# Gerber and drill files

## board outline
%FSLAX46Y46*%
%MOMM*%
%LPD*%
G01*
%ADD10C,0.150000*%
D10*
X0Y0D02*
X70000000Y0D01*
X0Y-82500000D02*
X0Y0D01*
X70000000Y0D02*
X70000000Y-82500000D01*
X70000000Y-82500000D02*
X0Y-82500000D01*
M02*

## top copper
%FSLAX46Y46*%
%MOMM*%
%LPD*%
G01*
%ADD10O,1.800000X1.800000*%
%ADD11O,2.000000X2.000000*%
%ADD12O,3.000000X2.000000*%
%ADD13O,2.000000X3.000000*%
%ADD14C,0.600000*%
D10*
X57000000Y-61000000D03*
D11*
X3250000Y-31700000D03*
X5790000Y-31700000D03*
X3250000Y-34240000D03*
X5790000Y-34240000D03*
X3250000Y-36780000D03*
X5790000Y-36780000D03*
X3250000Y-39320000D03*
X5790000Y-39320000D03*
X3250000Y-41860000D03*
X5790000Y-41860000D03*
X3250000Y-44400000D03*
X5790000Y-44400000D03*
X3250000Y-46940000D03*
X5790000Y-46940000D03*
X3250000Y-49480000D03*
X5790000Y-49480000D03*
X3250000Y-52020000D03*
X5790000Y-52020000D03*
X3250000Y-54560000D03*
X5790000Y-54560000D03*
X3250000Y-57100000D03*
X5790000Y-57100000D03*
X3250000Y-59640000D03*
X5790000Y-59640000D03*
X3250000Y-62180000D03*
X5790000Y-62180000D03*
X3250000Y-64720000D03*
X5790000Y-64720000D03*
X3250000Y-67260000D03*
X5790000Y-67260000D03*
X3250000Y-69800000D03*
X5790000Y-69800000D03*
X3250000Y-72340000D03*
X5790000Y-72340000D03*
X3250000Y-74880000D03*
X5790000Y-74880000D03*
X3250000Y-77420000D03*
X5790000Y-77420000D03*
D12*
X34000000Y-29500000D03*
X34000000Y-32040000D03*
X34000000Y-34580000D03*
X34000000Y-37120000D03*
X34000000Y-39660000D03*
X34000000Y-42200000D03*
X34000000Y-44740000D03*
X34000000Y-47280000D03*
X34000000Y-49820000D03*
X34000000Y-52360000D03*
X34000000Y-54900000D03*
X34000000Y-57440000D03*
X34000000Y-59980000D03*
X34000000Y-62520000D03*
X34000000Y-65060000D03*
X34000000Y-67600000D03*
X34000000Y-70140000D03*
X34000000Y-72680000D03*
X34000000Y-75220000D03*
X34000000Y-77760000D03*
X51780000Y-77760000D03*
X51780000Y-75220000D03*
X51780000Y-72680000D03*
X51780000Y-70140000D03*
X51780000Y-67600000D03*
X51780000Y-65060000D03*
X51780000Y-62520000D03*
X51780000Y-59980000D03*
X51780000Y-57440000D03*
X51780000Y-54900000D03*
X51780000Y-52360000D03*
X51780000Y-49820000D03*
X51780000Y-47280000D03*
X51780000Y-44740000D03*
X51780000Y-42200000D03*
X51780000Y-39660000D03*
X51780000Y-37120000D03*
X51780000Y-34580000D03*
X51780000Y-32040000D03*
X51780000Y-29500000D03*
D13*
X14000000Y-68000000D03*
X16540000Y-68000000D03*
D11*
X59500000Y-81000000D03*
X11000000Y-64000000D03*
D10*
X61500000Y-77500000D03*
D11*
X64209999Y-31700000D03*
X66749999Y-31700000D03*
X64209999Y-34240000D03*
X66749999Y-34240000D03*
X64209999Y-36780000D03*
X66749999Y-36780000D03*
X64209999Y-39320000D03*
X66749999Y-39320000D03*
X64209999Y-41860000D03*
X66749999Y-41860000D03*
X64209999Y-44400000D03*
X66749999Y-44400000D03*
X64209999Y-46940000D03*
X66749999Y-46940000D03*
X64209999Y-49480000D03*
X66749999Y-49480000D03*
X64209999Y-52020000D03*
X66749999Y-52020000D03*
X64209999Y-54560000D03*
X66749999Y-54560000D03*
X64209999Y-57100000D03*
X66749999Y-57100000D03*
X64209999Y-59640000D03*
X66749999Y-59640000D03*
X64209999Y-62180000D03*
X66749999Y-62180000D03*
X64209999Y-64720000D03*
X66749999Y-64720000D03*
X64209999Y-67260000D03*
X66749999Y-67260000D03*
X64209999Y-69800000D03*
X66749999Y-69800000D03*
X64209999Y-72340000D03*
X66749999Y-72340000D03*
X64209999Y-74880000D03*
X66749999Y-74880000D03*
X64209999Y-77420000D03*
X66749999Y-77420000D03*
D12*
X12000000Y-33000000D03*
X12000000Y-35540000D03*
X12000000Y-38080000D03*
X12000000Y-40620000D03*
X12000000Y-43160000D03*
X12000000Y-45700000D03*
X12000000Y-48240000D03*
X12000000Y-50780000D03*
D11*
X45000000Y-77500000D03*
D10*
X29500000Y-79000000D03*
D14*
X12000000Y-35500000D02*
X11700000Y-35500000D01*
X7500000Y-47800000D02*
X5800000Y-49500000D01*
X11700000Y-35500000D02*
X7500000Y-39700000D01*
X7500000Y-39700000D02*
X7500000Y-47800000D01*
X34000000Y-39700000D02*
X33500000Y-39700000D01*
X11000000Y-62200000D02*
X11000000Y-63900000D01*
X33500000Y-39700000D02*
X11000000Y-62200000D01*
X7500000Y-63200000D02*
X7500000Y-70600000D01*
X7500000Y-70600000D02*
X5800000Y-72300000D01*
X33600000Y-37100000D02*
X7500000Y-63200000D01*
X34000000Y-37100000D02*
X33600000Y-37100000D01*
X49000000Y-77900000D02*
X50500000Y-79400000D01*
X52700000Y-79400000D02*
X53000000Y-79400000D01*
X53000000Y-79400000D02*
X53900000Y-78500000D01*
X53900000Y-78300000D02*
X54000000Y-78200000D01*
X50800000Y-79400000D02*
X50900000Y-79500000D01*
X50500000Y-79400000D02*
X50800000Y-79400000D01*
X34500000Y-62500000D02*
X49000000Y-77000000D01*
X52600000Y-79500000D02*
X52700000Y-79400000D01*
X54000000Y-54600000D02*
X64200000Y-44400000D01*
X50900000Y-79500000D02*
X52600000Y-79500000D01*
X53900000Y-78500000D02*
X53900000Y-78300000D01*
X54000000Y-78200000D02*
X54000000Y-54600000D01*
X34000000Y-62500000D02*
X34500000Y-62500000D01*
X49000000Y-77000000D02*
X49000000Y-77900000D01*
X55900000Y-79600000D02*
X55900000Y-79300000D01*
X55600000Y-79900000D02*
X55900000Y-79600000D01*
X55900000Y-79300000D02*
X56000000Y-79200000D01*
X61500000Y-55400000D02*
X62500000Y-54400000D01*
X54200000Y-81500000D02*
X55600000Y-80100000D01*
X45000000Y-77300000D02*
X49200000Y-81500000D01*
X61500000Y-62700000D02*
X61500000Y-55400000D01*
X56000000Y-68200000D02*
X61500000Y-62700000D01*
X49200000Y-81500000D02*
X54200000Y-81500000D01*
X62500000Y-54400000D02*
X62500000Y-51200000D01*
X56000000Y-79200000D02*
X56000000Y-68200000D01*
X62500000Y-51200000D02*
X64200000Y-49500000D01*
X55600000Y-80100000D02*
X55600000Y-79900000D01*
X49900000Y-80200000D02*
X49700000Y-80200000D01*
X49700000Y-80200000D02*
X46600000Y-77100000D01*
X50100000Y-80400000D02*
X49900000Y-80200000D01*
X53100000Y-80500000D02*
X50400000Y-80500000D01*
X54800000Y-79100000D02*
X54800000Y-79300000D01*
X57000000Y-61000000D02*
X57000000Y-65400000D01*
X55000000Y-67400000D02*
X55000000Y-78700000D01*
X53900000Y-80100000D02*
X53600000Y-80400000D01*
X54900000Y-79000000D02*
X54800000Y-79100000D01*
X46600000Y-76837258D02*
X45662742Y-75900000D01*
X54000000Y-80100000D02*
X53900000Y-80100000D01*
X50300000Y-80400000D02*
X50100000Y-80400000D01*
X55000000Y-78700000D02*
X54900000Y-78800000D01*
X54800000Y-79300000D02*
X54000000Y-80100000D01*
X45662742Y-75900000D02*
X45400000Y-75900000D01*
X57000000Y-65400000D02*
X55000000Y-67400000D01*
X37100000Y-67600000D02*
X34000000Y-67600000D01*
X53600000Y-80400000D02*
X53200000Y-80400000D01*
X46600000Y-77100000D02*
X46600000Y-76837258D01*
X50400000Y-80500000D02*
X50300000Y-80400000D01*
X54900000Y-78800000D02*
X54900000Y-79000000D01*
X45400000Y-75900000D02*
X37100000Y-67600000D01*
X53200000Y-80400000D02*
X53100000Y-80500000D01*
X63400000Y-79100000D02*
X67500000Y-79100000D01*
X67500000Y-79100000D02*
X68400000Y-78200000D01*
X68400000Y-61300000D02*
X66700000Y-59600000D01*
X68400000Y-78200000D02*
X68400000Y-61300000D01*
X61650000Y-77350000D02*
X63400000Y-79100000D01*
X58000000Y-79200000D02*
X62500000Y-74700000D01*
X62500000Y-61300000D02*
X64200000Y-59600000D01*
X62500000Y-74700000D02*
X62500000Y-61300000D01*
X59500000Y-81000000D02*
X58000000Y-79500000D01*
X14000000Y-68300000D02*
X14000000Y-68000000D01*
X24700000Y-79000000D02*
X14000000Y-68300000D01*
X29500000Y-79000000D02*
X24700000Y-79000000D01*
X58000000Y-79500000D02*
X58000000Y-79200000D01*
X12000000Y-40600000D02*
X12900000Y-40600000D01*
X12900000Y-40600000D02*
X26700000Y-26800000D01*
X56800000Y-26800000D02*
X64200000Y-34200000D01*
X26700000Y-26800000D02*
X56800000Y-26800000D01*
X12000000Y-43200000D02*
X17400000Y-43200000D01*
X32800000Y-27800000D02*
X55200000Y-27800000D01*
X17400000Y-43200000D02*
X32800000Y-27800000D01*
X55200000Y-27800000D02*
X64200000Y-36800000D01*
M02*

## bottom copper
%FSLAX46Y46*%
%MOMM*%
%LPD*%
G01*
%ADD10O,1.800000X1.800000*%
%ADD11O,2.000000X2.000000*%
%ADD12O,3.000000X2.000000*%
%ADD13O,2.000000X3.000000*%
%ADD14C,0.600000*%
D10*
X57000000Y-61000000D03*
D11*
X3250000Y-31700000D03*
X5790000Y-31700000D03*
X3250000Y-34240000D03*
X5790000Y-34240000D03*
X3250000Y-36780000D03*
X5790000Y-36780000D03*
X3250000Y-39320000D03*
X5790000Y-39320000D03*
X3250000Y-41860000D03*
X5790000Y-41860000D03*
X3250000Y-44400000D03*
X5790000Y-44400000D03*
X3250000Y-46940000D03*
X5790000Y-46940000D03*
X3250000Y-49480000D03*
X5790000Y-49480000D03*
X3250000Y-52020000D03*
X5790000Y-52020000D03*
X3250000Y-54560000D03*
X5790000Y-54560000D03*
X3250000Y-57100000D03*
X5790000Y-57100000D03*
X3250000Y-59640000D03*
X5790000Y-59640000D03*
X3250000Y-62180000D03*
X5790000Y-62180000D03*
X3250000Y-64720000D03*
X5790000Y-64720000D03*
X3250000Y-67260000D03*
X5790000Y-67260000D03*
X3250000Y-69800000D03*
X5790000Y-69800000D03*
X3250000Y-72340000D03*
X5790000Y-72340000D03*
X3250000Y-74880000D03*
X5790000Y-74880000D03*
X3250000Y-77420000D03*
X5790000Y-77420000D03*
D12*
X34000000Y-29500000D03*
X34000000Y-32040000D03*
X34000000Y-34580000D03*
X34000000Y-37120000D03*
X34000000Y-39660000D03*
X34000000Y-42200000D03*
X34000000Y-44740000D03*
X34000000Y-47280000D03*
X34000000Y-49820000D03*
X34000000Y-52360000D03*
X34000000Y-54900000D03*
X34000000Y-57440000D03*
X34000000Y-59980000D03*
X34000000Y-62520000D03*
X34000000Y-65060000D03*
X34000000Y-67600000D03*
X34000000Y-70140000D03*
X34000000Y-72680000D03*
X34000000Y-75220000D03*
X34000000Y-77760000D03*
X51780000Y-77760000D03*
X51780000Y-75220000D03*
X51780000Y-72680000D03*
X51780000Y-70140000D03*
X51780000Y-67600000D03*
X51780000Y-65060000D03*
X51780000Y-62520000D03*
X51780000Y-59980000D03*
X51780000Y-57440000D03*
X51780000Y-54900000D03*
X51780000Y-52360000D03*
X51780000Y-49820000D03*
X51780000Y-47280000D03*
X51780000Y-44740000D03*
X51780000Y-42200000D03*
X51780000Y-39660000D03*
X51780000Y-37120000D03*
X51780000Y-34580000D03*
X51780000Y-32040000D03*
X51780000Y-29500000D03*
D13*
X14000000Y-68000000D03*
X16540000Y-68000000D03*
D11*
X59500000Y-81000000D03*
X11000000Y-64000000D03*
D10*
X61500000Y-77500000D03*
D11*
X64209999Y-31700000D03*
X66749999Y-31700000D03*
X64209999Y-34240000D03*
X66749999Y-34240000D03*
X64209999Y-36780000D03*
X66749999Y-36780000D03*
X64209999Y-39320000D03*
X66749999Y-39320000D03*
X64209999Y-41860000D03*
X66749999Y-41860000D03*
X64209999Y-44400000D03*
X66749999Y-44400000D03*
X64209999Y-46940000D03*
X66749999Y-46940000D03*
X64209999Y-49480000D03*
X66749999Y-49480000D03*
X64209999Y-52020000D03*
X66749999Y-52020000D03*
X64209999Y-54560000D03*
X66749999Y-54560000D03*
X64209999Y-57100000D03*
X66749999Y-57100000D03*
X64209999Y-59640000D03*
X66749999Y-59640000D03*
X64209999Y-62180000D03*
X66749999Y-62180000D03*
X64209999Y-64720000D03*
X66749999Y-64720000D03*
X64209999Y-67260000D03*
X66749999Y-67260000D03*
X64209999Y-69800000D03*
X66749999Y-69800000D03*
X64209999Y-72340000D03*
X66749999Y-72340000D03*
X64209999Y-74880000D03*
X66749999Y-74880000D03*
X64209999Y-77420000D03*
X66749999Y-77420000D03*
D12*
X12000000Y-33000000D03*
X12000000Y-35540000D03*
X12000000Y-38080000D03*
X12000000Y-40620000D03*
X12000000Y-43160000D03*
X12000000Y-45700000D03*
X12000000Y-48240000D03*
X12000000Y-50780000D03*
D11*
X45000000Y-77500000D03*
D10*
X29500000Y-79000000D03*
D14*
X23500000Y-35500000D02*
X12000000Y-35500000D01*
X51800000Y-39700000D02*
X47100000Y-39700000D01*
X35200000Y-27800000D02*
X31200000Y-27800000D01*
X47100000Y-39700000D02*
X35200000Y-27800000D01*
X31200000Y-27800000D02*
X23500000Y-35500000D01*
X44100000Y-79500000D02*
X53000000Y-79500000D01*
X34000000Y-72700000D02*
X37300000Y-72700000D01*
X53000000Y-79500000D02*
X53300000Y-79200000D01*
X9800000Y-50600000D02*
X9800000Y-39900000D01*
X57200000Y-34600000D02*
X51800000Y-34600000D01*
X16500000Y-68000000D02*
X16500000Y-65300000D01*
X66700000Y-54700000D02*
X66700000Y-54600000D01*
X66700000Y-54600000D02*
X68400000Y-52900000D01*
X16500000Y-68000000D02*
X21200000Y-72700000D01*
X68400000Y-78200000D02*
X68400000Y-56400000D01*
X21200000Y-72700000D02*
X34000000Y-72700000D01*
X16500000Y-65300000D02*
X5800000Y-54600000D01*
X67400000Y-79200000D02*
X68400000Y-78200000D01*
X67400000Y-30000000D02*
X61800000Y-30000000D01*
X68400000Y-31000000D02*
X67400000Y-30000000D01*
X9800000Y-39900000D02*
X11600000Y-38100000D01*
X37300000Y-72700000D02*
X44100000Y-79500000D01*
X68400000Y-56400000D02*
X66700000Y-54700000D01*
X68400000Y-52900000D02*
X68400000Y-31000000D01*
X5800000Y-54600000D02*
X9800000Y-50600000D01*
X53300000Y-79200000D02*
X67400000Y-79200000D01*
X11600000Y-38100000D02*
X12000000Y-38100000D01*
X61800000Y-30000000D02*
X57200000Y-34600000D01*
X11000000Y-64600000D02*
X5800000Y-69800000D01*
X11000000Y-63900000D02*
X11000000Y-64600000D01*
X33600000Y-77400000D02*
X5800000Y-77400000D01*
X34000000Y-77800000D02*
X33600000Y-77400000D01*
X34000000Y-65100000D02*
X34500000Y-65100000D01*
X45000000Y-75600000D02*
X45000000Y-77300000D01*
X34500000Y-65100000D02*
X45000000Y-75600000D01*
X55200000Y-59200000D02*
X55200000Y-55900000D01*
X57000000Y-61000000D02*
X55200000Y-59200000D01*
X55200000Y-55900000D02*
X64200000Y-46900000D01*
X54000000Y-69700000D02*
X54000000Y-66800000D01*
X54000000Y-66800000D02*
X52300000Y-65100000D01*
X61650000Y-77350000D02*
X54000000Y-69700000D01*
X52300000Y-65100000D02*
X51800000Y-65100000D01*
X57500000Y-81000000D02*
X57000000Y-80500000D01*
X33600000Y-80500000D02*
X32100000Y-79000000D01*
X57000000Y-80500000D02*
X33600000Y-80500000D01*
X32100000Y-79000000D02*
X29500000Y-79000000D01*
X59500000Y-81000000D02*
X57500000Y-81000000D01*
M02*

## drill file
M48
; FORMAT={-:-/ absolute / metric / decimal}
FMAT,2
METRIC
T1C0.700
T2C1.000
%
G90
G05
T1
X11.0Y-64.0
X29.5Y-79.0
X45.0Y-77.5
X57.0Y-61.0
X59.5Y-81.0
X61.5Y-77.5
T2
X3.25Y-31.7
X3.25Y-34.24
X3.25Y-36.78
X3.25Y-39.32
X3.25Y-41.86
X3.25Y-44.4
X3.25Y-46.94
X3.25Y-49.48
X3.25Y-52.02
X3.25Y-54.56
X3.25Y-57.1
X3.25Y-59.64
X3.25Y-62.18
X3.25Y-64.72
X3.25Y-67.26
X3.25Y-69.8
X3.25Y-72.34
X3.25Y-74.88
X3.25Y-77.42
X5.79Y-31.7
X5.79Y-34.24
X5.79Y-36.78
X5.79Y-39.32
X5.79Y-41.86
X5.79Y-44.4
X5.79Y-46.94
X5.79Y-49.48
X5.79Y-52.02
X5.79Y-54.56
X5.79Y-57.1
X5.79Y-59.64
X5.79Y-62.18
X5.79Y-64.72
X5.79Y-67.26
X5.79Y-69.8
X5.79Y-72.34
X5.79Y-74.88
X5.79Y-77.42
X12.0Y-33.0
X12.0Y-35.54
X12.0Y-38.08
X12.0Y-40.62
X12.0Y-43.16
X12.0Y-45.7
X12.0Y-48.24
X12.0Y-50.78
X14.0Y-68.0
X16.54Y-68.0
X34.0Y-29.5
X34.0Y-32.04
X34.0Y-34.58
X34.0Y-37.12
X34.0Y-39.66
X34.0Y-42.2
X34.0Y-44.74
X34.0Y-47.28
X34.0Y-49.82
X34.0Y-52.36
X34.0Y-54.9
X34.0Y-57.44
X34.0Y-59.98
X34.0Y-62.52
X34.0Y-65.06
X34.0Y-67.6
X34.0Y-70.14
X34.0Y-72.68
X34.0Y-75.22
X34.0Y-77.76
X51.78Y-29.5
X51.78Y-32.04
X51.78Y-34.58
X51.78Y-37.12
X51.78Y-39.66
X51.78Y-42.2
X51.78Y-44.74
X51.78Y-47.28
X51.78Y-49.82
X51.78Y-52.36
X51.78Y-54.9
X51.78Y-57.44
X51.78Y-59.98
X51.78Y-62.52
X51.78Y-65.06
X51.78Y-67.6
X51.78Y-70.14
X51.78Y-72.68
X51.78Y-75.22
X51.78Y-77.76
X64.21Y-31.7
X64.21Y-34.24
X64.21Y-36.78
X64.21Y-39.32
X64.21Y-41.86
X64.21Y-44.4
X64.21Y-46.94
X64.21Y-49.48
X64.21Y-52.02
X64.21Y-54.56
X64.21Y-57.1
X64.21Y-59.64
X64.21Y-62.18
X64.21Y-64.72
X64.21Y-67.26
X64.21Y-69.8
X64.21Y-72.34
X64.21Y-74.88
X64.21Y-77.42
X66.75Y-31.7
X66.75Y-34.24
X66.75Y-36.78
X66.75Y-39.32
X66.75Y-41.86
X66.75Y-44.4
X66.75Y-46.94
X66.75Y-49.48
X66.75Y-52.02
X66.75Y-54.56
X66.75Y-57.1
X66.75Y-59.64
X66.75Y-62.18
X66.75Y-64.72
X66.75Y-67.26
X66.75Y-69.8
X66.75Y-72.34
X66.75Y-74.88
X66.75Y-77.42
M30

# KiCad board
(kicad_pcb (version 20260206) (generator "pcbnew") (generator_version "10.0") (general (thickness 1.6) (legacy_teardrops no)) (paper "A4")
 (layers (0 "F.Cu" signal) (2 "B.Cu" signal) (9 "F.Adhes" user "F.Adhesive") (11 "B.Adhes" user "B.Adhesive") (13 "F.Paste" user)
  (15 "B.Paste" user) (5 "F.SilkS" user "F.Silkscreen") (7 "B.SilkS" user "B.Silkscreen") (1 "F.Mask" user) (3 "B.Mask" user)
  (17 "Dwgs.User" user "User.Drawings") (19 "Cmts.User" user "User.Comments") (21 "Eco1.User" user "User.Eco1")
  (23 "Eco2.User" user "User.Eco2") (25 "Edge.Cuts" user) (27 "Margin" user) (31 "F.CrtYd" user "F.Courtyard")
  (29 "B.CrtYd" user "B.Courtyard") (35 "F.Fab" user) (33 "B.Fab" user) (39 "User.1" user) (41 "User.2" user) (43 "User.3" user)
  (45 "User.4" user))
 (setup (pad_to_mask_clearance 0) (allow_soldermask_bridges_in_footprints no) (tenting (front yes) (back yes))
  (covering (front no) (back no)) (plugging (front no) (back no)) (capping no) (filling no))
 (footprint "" (layer "F.Cu") (at 57 61)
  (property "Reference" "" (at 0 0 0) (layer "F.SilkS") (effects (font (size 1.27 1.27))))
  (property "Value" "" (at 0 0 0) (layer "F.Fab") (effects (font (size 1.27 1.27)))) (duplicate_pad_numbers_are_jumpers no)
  (pad "2" thru_hole oval (at 0 0) (size 1.8 1.8) (drill 0.7) (layers "*.Cu" "*.Mask") (remove_unused_layers no)))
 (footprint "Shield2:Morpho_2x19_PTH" (layer "F.Cu") (at 3.25 31.7)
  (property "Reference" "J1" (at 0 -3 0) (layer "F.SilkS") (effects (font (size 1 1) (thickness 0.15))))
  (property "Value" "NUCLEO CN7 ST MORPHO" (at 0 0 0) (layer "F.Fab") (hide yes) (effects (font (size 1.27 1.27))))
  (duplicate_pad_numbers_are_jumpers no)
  (pad "1" thru_hole oval (at 0 0) (size 2 2) (drill 1) (layers "*.Cu") (remove_unused_layers no) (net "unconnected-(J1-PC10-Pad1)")
   (thermal_bridge_angle 45))
  (pad "2" thru_hole oval (at 2.54 0) (size 2 2) (drill 1) (layers "*.Cu") (remove_unused_layers no) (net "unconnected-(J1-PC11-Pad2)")
   (thermal_bridge_angle 45))
  (pad "3" thru_hole oval (at 0 2.54) (size 2 2) (drill 1) (layers "*.Cu") (remove_unused_layers no) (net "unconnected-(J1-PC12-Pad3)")
   (thermal_bridge_angle 45))
  (pad "4" thru_hole oval (at 2.54 2.54) (size 2 2) (drill 1) (layers "*.Cu") (remove_unused_layers no) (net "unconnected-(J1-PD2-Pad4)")
   (thermal_bridge_angle 45))
  (pad "5" thru_hole oval (at 0 5.08) (size 2 2) (drill 1) (layers "*.Cu") (remove_unused_layers no) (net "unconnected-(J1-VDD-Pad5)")
   (thermal_bridge_angle 45))
  (pad "6" thru_hole oval (at 2.54 5.08) (size 2 2) (drill 1) (layers "*.Cu") (remove_unused_layers no) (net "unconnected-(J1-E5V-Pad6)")
   (thermal_bridge_angle 45))
  (pad "7" thru_hole oval (at 0 7.62) (size 2 2) (drill 1) (layers "*.Cu") (remove_unused_layers no) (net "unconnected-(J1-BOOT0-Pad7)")
   (thermal_bridge_angle 45))
  (pad "8" thru_hole oval (at 2.54 7.62) (size 2 2) (drill 1) (layers "*.Cu") (remove_unused_layers no) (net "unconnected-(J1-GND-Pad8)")
   (thermal_bridge_angle 45))
  (pad "9" thru_hole oval (at 0 10.16) (size 2 2) (drill 1) (layers "*.Cu") (remove_unused_layers no) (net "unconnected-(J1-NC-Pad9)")
   (thermal_bridge_angle 45))
  (pad "10" thru_hole oval (at 2.54 10.16) (size 2 2) (drill 1) (layers "*.Cu") (remove_unused_layers no) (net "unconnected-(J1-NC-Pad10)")
   (thermal_bridge_angle 45))
  (pad "11" thru_hole oval (at 0 12.7) (size 2 2) (drill 1) (layers "*.Cu") (remove_unused_layers no) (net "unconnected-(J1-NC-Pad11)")
   (thermal_bridge_angle 45))
  (pad "12" thru_hole oval (at 2.54 12.7) (size 2 2) (drill 1) (layers "*.Cu") (remove_unused_layers no)
   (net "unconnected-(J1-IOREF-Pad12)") (thermal_bridge_angle 45))
  (pad "13" thru_hole oval (at 0 15.24) (size 2 2) (drill 1) (layers "*.Cu") (remove_unused_layers no) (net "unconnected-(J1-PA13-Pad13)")
   (thermal_bridge_angle 45))
  (pad "14" thru_hole oval (at 2.54 15.24) (size 2 2) (drill 1) (layers "*.Cu") (remove_unused_layers no)
   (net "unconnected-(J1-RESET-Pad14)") (thermal_bridge_angle 45))
  (pad "15" thru_hole oval (at 0 17.78) (size 2 2) (drill 1) (layers "*.Cu") (remove_unused_layers no) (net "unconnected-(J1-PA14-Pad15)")
   (thermal_bridge_angle 45))
  (pad "16" thru_hole oval (at 2.54 17.78) (size 2 2) (drill 1) (layers "*.Cu") (remove_unused_layers no) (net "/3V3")
   (thermal_bridge_angle 45))
  (pad "17" thru_hole oval (at 0 20.32) (size 2 2) (drill 1) (layers "*.Cu") (remove_unused_layers no) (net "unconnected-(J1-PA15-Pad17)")
   (thermal_bridge_angle 45))
  (pad "18" thru_hole oval (at 2.54 20.32) (size 2 2) (drill 1) (layers "*.Cu") (remove_unused_layers no) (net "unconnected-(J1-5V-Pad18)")
   (thermal_bridge_angle 45))
  (pad "19" thru_hole oval (at 0 22.86) (size 2 2) (drill 1) (layers "*.Cu") (remove_unused_layers no) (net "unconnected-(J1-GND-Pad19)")
   (thermal_bridge_angle 45))
  (pad "20" thru_hole oval (at 2.54 22.86) (size 2 2) (drill 1) (layers "*.Cu") (remove_unused_layers no) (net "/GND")
   (thermal_bridge_angle 45))
  (pad "21" thru_hole oval (at 0 25.4) (size 2 2) (drill 1) (layers "*.Cu") (remove_unused_layers no) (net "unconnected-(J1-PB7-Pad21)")
   (thermal_bridge_angle 45))
  (pad "22" thru_hole oval (at 2.54 25.4) (size 2 2) (drill 1) (layers "*.Cu") (remove_unused_layers no) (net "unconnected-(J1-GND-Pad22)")
   (thermal_bridge_angle 45))
  (pad "23" thru_hole oval (at 0 27.94) (size 2 2) (drill 1) (layers "*.Cu") (remove_unused_layers no) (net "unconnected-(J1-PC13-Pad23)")
   (thermal_bridge_angle 45))
  (pad "24" thru_hole oval (at 2.54 27.94) (size 2 2) (drill 1) (layers "*.Cu") (remove_unused_layers no) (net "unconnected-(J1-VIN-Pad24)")
   (thermal_bridge_angle 45))
  (pad "25" thru_hole oval (at 0 30.48) (size 2 2) (drill 1) (layers "*.Cu") (remove_unused_layers no) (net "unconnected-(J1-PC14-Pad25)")
   (thermal_bridge_angle 45))
  (pad "26" thru_hole oval (at 2.54 30.48) (size 2 2) (drill 1) (layers "*.Cu") (remove_unused_layers no) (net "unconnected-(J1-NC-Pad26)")
   (thermal_bridge_angle 45))
  (pad "27" thru_hole oval (at 0 33.02) (size 2 2) (drill 1) (layers "*.Cu") (remove_unused_layers no) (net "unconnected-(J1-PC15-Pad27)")
   (thermal_bridge_angle 45))
  (pad "28" thru_hole oval (at 2.54 33.02) (size 2 2) (drill 1) (layers "*.Cu") (remove_unused_layers no) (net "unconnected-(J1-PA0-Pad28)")
   (thermal_bridge_angle 45))
  (pad "29" thru_hole oval (at 0 35.56) (size 2 2) (drill 1) (layers "*.Cu") (remove_unused_layers no) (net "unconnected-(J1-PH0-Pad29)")
   (thermal_bridge_angle 45))
  (pad "30" thru_hole oval (at 2.54 35.56) (size 2 2) (drill 1) (layers "*.Cu") (remove_unused_layers no) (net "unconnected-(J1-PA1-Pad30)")
   (thermal_bridge_angle 45))
  (pad "31" thru_hole oval (at 0 38.1) (size 2 2) (drill 1) (layers "*.Cu") (remove_unused_layers no) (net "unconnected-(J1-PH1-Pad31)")
   (thermal_bridge_angle 45))
  (pad "32" thru_hole oval (at 2.54 38.1) (size 2 2) (drill 1) (layers "*.Cu") (remove_unused_layers no) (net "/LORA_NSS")
   (thermal_bridge_angle 45))
  (pad "33" thru_hole oval (at 0 40.64) (size 2 2) (drill 1) (layers "*.Cu") (remove_unused_layers no) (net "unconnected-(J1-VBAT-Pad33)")
   (thermal_bridge_angle 45))
  (pad "34" thru_hole oval (at 2.54 40.64) (size 2 2) (drill 1) (layers "*.Cu") (remove_unused_layers no) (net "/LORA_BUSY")
   (thermal_bridge_angle 45))
  (pad "35" thru_hole oval (at 0 43.18) (size 2 2) (drill 1) (layers "*.Cu") (remove_unused_layers no) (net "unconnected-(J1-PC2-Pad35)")
   (thermal_bridge_angle 45))
  (pad "36" thru_hole oval (at 2.54 43.18) (size 2 2) (drill 1) (layers "*.Cu") (remove_unused_layers no)
   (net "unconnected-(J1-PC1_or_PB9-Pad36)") (thermal_bridge_angle 45))
  (pad "37" thru_hole oval (at 0 45.72) (size 2 2) (drill 1) (layers "*.Cu") (remove_unused_layers no) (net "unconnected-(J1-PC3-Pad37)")
   (thermal_bridge_angle 45))
  (pad "38" thru_hole oval (at 2.54 45.72) (size 2 2) (drill 1) (layers "*.Cu") (remove_unused_layers no) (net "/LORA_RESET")
   (thermal_bridge_angle 45)))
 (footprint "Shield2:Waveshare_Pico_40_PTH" (layer "F.Cu") (at 34 29.5)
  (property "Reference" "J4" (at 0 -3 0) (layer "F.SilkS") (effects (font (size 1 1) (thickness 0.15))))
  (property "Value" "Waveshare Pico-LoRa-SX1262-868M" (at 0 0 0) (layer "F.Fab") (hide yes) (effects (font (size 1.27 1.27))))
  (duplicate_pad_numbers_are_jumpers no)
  (pad "1" thru_hole oval (at 0 0) (size 3 2) (drill 1) (layers "*.Cu") (remove_unused_layers no) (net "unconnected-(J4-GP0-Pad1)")
   (thermal_bridge_angle 45))
  (pad "2" thru_hole oval (at 0 2.54) (size 3 2) (drill 1) (layers "*.Cu") (remove_unused_layers no) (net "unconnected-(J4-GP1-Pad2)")
   (thermal_bridge_angle 45))
  (pad "3" thru_hole oval (at 0 5.08) (size 3 2) (drill 1) (layers "*.Cu") (remove_unused_layers no) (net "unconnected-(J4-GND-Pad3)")
   (thermal_bridge_angle 45))
  (pad "4" thru_hole oval (at 0 7.62) (size 3 2) (drill 1) (layers "*.Cu") (remove_unused_layers no) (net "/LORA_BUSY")
   (thermal_bridge_angle 45))
  (pad "5" thru_hole oval (at 0 10.16) (size 3 2) (drill 1) (layers "*.Cu") (remove_unused_layers no) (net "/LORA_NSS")
   (thermal_bridge_angle 45))
  (pad "6" thru_hole oval (at 0 12.7) (size 3 2) (drill 1) (layers "*.Cu") (remove_unused_layers no) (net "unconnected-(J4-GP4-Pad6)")
   (thermal_bridge_angle 45))
  (pad "7" thru_hole oval (at 0 15.24) (size 3 2) (drill 1) (layers "*.Cu") (remove_unused_layers no) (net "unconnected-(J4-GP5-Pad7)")
   (thermal_bridge_angle 45))
  (pad "8" thru_hole oval (at 0 17.78) (size 3 2) (drill 1) (layers "*.Cu") (remove_unused_layers no) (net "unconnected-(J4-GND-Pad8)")
   (thermal_bridge_angle 45))
  (pad "9" thru_hole oval (at 0 20.32) (size 3 2) (drill 1) (layers "*.Cu") (remove_unused_layers no) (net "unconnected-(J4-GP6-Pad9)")
   (thermal_bridge_angle 45))
  (pad "10" thru_hole oval (at 0 22.86) (size 3 2) (drill 1) (layers "*.Cu") (remove_unused_layers no) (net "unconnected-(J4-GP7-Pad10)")
   (thermal_bridge_angle 45))
  (pad "11" thru_hole oval (at 0 25.4) (size 3 2) (drill 1) (layers "*.Cu") (remove_unused_layers no) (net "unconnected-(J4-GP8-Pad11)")
   (thermal_bridge_angle 45))
  (pad "12" thru_hole oval (at 0 27.94) (size 3 2) (drill 1) (layers "*.Cu") (remove_unused_layers no) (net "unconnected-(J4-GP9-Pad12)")
   (thermal_bridge_angle 45))
  (pad "13" thru_hole oval (at 0 30.48) (size 3 2) (drill 1) (layers "*.Cu") (remove_unused_layers no) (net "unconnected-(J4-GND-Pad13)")
   (thermal_bridge_angle 45))
  (pad "14" thru_hole oval (at 0 33.02) (size 3 2) (drill 1) (layers "*.Cu") (remove_unused_layers no) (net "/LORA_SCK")
   (thermal_bridge_angle 45))
  (pad "15" thru_hole oval (at 0 35.56) (size 3 2) (drill 1) (layers "*.Cu") (remove_unused_layers no) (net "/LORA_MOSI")
   (thermal_bridge_angle 45))
  (pad "16" thru_hole oval (at 0 38.1) (size 3 2) (drill 1) (layers "*.Cu") (remove_unused_layers no) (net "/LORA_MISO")
   (thermal_bridge_angle 45))
  (pad "17" thru_hole oval (at 0 40.64) (size 3 2) (drill 1) (layers "*.Cu") (remove_unused_layers no) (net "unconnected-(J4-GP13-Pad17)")
   (thermal_bridge_angle 45))
  (pad "18" thru_hole oval (at 0 43.18) (size 3 2) (drill 1) (layers "*.Cu") (remove_unused_layers no) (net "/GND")
   (thermal_bridge_angle 45))
  (pad "19" thru_hole oval (at 0 45.72) (size 3 2) (drill 1) (layers "*.Cu") (remove_unused_layers no) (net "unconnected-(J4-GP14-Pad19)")
   (thermal_bridge_angle 45))
  (pad "20" thru_hole oval (at 0 48.26) (size 3 2) (drill 1) (layers "*.Cu") (remove_unused_layers no) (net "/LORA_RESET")
   (thermal_bridge_angle 45))
  (pad "21" thru_hole oval (at 17.78 48.26) (size 3 2) (drill 1) (layers "*.Cu") (remove_unused_layers no)
   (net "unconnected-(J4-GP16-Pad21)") (thermal_bridge_angle 45))
  (pad "22" thru_hole oval (at 17.78 45.72) (size 3 2) (drill 1) (layers "*.Cu") (remove_unused_layers no)
   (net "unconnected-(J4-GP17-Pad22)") (thermal_bridge_angle 45))
  (pad "23" thru_hole oval (at 17.78 43.18) (size 3 2) (drill 1) (layers "*.Cu") (remove_unused_layers no)
   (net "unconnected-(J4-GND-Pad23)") (thermal_bridge_angle 45))
  (pad "24" thru_hole oval (at 17.78 40.64) (size 3 2) (drill 1) (layers "*.Cu") (remove_unused_layers no)
   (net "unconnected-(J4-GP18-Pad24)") (thermal_bridge_angle 45))
  (pad "25" thru_hole oval (at 17.78 38.1) (size 3 2) (drill 1) (layers "*.Cu") (remove_unused_layers no)
   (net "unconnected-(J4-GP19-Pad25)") (thermal_bridge_angle 45))
  (pad "26" thru_hole oval (at 17.78 35.56) (size 3 2) (drill 1) (layers "*.Cu") (remove_unused_layers no) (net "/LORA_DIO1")
   (thermal_bridge_angle 45))
  (pad "27" thru_hole oval (at 17.78 33.02) (size 3 2) (drill 1) (layers "*.Cu") (remove_unused_layers no)
   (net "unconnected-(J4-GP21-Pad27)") (thermal_bridge_angle 45))
  (pad "28" thru_hole oval (at 17.78 30.48) (size 3 2) (drill 1) (layers "*.Cu") (remove_unused_layers no)
   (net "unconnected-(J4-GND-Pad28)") (thermal_bridge_angle 45))
  (pad "29" thru_hole oval (at 17.78 27.94) (size 3 2) (drill 1) (layers "*.Cu") (remove_unused_layers no)
   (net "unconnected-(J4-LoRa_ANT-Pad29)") (thermal_bridge_angle 45))
  (pad "30" thru_hole oval (at 17.78 25.4) (size 3 2) (drill 1) (layers "*.Cu") (remove_unused_layers no) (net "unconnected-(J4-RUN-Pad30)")
   (thermal_bridge_angle 45))
  (pad "31" thru_hole oval (at 17.78 22.86) (size 3 2) (drill 1) (layers "*.Cu") (remove_unused_layers no)
   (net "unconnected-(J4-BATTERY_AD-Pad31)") (thermal_bridge_angle 45))
  (pad "32" thru_hole oval (at 17.78 20.32) (size 3 2) (drill 1) (layers "*.Cu") (remove_unused_layers no)
   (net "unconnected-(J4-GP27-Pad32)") (thermal_bridge_angle 45))
  (pad "33" thru_hole oval (at 17.78 17.78) (size 3 2) (drill 1) (layers "*.Cu") (remove_unused_layers no)
   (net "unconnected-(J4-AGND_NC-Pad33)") (thermal_bridge_angle 45))
  (pad "34" thru_hole oval (at 17.78 15.24) (size 3 2) (drill 1) (layers "*.Cu") (remove_unused_layers no)
   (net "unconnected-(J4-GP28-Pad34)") (thermal_bridge_angle 45))
  (pad "35" thru_hole oval (at 17.78 12.7) (size 3 2) (drill 1) (layers "*.Cu") (remove_unused_layers no)
   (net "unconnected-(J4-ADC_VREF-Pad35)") (thermal_bridge_angle 45))
  (pad "36" thru_hole oval (at 17.78 10.16) (size 3 2) (drill 1) (layers "*.Cu") (remove_unused_layers no) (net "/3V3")
   (thermal_bridge_angle 45))
  (pad "37" thru_hole oval (at 17.78 7.62) (size 3 2) (drill 1) (layers "*.Cu") (remove_unused_layers no)
   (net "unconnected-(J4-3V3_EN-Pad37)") (thermal_bridge_angle 45))
  (pad "38" thru_hole oval (at 17.78 5.08) (size 3 2) (drill 1) (layers "*.Cu") (remove_unused_layers no) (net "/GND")
   (thermal_bridge_angle 45))
  (pad "39" thru_hole oval (at 17.78 2.54) (size 3 2) (drill 1) (layers "*.Cu") (remove_unused_layers no)
   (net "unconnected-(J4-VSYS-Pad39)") (thermal_bridge_angle 45))
  (pad "40" thru_hole oval (at 17.78 0) (size 3 2) (drill 1) (layers "*.Cu") (remove_unused_layers no) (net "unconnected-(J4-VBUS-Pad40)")
   (thermal_bridge_angle 45)))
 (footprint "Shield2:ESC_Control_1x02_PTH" (layer "F.Cu") (at 14 68)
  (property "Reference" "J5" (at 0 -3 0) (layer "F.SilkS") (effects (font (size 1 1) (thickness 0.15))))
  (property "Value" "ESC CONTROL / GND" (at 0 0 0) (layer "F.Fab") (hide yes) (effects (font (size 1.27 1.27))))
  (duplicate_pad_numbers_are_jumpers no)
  (pad "1" thru_hole oval (at 0 0) (size 2 3) (drill 1) (layers "*.Cu") (remove_unused_layers no) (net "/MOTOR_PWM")
   (thermal_bridge_angle 45))
  (pad "2" thru_hole oval (at 2.54 0) (size 2 3) (drill 1) (layers "*.Cu") (remove_unused_layers no) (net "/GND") (thermal_bridge_angle 45)))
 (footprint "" (layer "F.Cu") (at 59.5 81)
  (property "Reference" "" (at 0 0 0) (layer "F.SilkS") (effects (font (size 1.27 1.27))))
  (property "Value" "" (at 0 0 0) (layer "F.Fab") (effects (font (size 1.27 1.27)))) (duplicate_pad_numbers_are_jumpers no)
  (pad "2" thru_hole oval (at 0 0) (size 2 2) (drill 0.7) (layers "*.Cu" "*.Mask") (remove_unused_layers no)))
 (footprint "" (layer "F.Cu") (at 11 64)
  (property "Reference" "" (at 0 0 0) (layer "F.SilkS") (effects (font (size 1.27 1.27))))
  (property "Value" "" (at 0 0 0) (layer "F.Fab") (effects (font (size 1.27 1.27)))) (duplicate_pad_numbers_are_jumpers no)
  (pad "2" thru_hole oval (at 0 0) (size 2 2) (drill 0.7) (layers "*.Cu" "*.Mask") (remove_unused_layers no)))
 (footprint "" (layer "F.Cu") (at 61.5 77.5)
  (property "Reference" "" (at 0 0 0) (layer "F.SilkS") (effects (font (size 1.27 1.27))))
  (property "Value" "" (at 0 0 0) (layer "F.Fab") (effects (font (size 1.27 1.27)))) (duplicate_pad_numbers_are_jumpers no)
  (pad "2" thru_hole oval (at 0 0) (size 1.8 1.8) (drill 0.7) (layers "*.Cu" "*.Mask") (remove_unused_layers no)))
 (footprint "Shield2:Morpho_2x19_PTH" (layer "F.Cu") (at 64.209999 31.7)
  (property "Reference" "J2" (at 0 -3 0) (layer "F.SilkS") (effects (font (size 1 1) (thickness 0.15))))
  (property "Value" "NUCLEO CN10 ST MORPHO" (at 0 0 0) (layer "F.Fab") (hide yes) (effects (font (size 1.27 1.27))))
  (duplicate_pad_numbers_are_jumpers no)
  (pad "1" thru_hole oval (at 0 0) (size 2 2) (drill 1) (layers "*.Cu") (remove_unused_layers no) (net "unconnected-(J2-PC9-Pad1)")
   (thermal_bridge_angle 45))
  (pad "2" thru_hole oval (at 2.54 0) (size 2 2) (drill 1) (layers "*.Cu") (remove_unused_layers no) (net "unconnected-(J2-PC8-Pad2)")
   (thermal_bridge_angle 45))
  (pad "3" thru_hole oval (at 0 2.54) (size 2 2) (drill 1) (layers "*.Cu") (remove_unused_layers no) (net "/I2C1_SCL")
   (thermal_bridge_angle 45))
  (pad "4" thru_hole oval (at 2.54 2.54) (size 2 2) (drill 1) (layers "*.Cu") (remove_unused_layers no) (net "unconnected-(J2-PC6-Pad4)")
   (thermal_bridge_angle 45))
  (pad "5" thru_hole oval (at 0 5.08) (size 2 2) (drill 1) (layers "*.Cu") (remove_unused_layers no) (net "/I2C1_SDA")
   (thermal_bridge_angle 45))
  (pad "6" thru_hole oval (at 2.54 5.08) (size 2 2) (drill 1) (layers "*.Cu") (remove_unused_layers no) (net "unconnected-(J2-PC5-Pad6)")
   (thermal_bridge_angle 45))
  (pad "7" thru_hole oval (at 0 7.62) (size 2 2) (drill 1) (layers "*.Cu") (remove_unused_layers no) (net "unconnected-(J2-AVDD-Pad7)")
   (thermal_bridge_angle 45))
  (pad "8" thru_hole oval (at 2.54 7.62) (size 2 2) (drill 1) (layers "*.Cu") (remove_unused_layers no) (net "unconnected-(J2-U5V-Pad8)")
   (thermal_bridge_angle 45))
  (pad "9" thru_hole oval (at 0 10.16) (size 2 2) (drill 1) (layers "*.Cu") (remove_unused_layers no) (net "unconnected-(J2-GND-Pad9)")
   (thermal_bridge_angle 45))
  (pad "10" thru_hole oval (at 2.54 10.16) (size 2 2) (drill 1) (layers "*.Cu") (remove_unused_layers no) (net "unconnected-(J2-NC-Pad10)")
   (thermal_bridge_angle 45))
  (pad "11" thru_hole oval (at 0 12.7) (size 2 2) (drill 1) (layers "*.Cu") (remove_unused_layers no) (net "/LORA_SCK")
   (thermal_bridge_angle 45))
  (pad "12" thru_hole oval (at 2.54 12.7) (size 2 2) (drill 1) (layers "*.Cu") (remove_unused_layers no) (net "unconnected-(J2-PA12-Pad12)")
   (thermal_bridge_angle 45))
  (pad "13" thru_hole oval (at 0 15.24) (size 2 2) (drill 1) (layers "*.Cu") (remove_unused_layers no) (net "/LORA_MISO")
   (thermal_bridge_angle 45))
  (pad "14" thru_hole oval (at 2.54 15.24) (size 2 2) (drill 1) (layers "*.Cu") (remove_unused_layers no)
   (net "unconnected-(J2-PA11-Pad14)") (thermal_bridge_angle 45))
  (pad "15" thru_hole oval (at 0 17.78) (size 2 2) (drill 1) (layers "*.Cu") (remove_unused_layers no) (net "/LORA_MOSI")
   (thermal_bridge_angle 45))
  (pad "16" thru_hole oval (at 2.54 17.78) (size 2 2) (drill 1) (layers "*.Cu") (remove_unused_layers no)
   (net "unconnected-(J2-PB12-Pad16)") (thermal_bridge_angle 45))
  (pad "17" thru_hole oval (at 0 20.32) (size 2 2) (drill 1) (layers "*.Cu") (remove_unused_layers no) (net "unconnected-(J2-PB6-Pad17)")
   (thermal_bridge_angle 45))
  (pad "18" thru_hole oval (at 2.54 20.32) (size 2 2) (drill 1) (layers "*.Cu") (remove_unused_layers no)
   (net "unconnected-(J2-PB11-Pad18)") (thermal_bridge_angle 45))
  (pad "19" thru_hole oval (at 0 22.86) (size 2 2) (drill 1) (layers "*.Cu") (remove_unused_layers no) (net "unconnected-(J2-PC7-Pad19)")
   (thermal_bridge_angle 45))
  (pad "20" thru_hole oval (at 2.54 22.86) (size 2 2) (drill 1) (layers "*.Cu") (remove_unused_layers no) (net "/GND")
   (thermal_bridge_angle 45))
  (pad "21" thru_hole oval (at 0 25.4) (size 2 2) (drill 1) (layers "*.Cu") (remove_unused_layers no) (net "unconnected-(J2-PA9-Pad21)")
   (thermal_bridge_angle 45))
  (pad "22" thru_hole oval (at 2.54 25.4) (size 2 2) (drill 1) (layers "*.Cu") (remove_unused_layers no) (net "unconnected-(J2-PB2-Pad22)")
   (thermal_bridge_angle 45))
  (pad "23" thru_hole oval (at 0 27.94) (size 2 2) (drill 1) (layers "*.Cu") (remove_unused_layers no) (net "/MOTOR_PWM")
   (thermal_bridge_angle 45))
  (pad "24" thru_hole oval (at 2.54 27.94) (size 2 2) (drill 1) (layers "*.Cu") (remove_unused_layers no) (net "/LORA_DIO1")
   (thermal_bridge_angle 45))
  (pad "25" thru_hole oval (at 0 30.48) (size 2 2) (drill 1) (layers "*.Cu") (remove_unused_layers no) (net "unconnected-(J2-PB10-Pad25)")
   (thermal_bridge_angle 45))
  (pad "26" thru_hole oval (at 2.54 30.48) (size 2 2) (drill 1) (layers "*.Cu") (remove_unused_layers no)
   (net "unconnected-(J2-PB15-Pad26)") (thermal_bridge_angle 45))
  (pad "27" thru_hole oval (at 0 33.02) (size 2 2) (drill 1) (layers "*.Cu") (remove_unused_layers no) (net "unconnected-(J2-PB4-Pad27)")
   (thermal_bridge_angle 45))
  (pad "28" thru_hole oval (at 2.54 33.02) (size 2 2) (drill 1) (layers "*.Cu") (remove_unused_layers no)
   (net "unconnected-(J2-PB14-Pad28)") (thermal_bridge_angle 45))
  (pad "29" thru_hole oval (at 0 35.56) (size 2 2) (drill 1) (layers "*.Cu") (remove_unused_layers no) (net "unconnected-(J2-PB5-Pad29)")
   (thermal_bridge_angle 45))
  (pad "30" thru_hole oval (at 2.54 35.56) (size 2 2) (drill 1) (layers "*.Cu") (remove_unused_layers no)
   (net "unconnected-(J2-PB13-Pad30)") (thermal_bridge_angle 45))
  (pad "31" thru_hole oval (at 0 38.1) (size 2 2) (drill 1) (layers "*.Cu") (remove_unused_layers no) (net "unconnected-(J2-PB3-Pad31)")
   (thermal_bridge_angle 45))
  (pad "32" thru_hole oval (at 2.54 38.1) (size 2 2) (drill 1) (layers "*.Cu") (remove_unused_layers no) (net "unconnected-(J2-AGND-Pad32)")
   (thermal_bridge_angle 45))
  (pad "33" thru_hole oval (at 0 40.64) (size 2 2) (drill 1) (layers "*.Cu") (remove_unused_layers no) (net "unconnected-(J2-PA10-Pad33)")
   (thermal_bridge_angle 45))
  (pad "34" thru_hole oval (at 2.54 40.64) (size 2 2) (drill 1) (layers "*.Cu") (remove_unused_layers no) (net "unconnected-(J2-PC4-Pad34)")
   (thermal_bridge_angle 45))
  (pad "35" thru_hole oval (at 0 43.18) (size 2 2) (drill 1) (layers "*.Cu") (remove_unused_layers no) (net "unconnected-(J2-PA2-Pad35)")
   (thermal_bridge_angle 45))
  (pad "36" thru_hole oval (at 2.54 43.18) (size 2 2) (drill 1) (layers "*.Cu") (remove_unused_layers no) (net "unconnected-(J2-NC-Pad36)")
   (thermal_bridge_angle 45))
  (pad "37" thru_hole oval (at 0 45.72) (size 2 2) (drill 1) (layers "*.Cu") (remove_unused_layers no) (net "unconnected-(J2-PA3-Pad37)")
   (thermal_bridge_angle 45))
  (pad "38" thru_hole oval (at 2.54 45.72) (size 2 2) (drill 1) (layers "*.Cu") (remove_unused_layers no) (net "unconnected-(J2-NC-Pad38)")
   (thermal_bridge_angle 45)))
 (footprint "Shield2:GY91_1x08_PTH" (layer "F.Cu") (at 12 33)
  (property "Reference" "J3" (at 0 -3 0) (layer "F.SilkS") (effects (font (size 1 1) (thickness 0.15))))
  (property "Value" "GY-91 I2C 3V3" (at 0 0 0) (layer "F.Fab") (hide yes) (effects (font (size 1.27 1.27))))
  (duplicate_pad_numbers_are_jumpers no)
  (pad "1" thru_hole oval (at 0 0) (size 3 2) (drill 1) (layers "*.Cu") (remove_unused_layers no) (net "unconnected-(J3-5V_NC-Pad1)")
   (thermal_bridge_angle 45))
  (pad "2" thru_hole oval (at 0 2.54) (size 3 2) (drill 1) (layers "*.Cu") (remove_unused_layers no) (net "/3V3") (thermal_bridge_angle 45))
  (pad "3" thru_hole oval (at 0 5.08) (size 3 2) (drill 1) (layers "*.Cu") (remove_unused_layers no) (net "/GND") (thermal_bridge_angle 45))
  (pad "4" thru_hole oval (at 0 7.62) (size 3 2) (drill 1) (layers "*.Cu") (remove_unused_layers no) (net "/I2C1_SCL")
   (thermal_bridge_angle 45))
  (pad "5" thru_hole oval (at 0 10.16) (size 3 2) (drill 1) (layers "*.Cu") (remove_unused_layers no) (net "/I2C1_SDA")
   (thermal_bridge_angle 45))
  (pad "6" thru_hole oval (at 0 12.7) (size 3 2) (drill 1) (layers "*.Cu") (remove_unused_layers no) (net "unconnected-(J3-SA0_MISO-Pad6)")
   (thermal_bridge_angle 45))
  (pad "7" thru_hole oval (at 0 15.24) (size 3 2) (drill 1) (layers "*.Cu") (remove_unused_layers no) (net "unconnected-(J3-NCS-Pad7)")
   (thermal_bridge_angle 45))
  (pad "8" thru_hole oval (at 0 17.78) (size 3 2) (drill 1) (layers "*.Cu") (remove_unused_layers no) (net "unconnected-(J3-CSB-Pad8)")
   (thermal_bridge_angle 45)))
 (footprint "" (layer "F.Cu") (at 45 77.5)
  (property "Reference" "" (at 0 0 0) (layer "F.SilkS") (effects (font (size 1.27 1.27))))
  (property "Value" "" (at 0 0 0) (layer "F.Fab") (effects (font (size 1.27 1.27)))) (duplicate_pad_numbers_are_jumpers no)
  (pad "2" thru_hole oval (at 0 0) (size 2 2) (drill 0.7) (layers "*.Cu" "*.Mask") (remove_unused_layers no)))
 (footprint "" (layer "F.Cu") (at 29.5 79)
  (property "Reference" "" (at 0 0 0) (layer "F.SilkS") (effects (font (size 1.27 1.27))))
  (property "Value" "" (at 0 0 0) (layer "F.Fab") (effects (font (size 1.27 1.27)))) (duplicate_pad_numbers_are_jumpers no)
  (pad "2" thru_hole oval (at 0 0) (size 1.8 1.8) (drill 0.7) (layers "*.Cu" "*.Mask") (remove_unused_layers no)))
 (gr_line (start 0 0) (end 70 0) (stroke (width 0.15) (type default)) (layer "Edge.Cuts"))
 (gr_line (start 0 82.5) (end 0 0) (stroke (width 0.15) (type default)) (layer "Edge.Cuts"))
 (gr_line (start 70 0) (end 70 82.5) (stroke (width 0.15) (type default)) (layer "Edge.Cuts"))
 (gr_line (start 70 82.5) (end 0 82.5) (stroke (width 0.15) (type default)) (layer "Edge.Cuts"))
 (segment (start 12 35.5) (end 11.7 35.5) (width 0.6) (layer "F.Cu") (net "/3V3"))
 (segment (start 7.5 47.8) (end 5.8 49.5) (width 0.6) (layer "F.Cu") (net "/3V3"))
 (segment (start 11.7 35.5) (end 7.5 39.7) (width 0.6) (layer "F.Cu") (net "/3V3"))
 (segment (start 7.5 39.7) (end 7.5 47.8) (width 0.6) (layer "F.Cu") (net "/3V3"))
 (segment (start 23.5 35.5) (end 12 35.5) (width 0.6) (layer "B.Cu") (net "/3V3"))
 (segment (start 51.8 39.7) (end 47.1 39.7) (width 0.6) (layer "B.Cu") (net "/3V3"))
 (segment (start 35.2 27.8) (end 31.2 27.8) (width 0.6) (layer "B.Cu") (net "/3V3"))
 (segment (start 47.1 39.7) (end 35.2 27.8) (width 0.6) (layer "B.Cu") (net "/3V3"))
 (segment (start 31.2 27.8) (end 23.5 35.5) (width 0.6) (layer "B.Cu") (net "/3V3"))
 (segment (start 44.1 79.5) (end 53 79.5) (width 0.6) (layer "B.Cu") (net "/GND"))
 (segment (start 34 72.7) (end 37.3 72.7) (width 0.6) (layer "B.Cu") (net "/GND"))
 (segment (start 53 79.5) (end 53.3 79.2) (width 0.6) (layer "B.Cu") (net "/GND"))
 (segment (start 9.8 50.6) (end 9.8 39.9) (width 0.6) (layer "B.Cu") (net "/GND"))
 (segment (start 57.2 34.6) (end 51.8 34.6) (width 0.6) (layer "B.Cu") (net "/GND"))
 (segment (start 16.5 68) (end 16.5 65.3) (width 0.6) (layer "B.Cu") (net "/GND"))
 (segment (start 66.7 54.7) (end 66.7 54.6) (width 0.6) (layer "B.Cu") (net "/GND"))
 (segment (start 66.7 54.6) (end 68.4 52.9) (width 0.6) (layer "B.Cu") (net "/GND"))
 (segment (start 16.5 68) (end 21.2 72.7) (width 0.6) (layer "B.Cu") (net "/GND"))
 (segment (start 68.4 78.2) (end 68.4 56.4) (width 0.6) (layer "B.Cu") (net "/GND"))
 (segment (start 21.2 72.7) (end 34 72.7) (width 0.6) (layer "B.Cu") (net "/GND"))
 (segment (start 16.5 65.3) (end 5.8 54.6) (width 0.6) (layer "B.Cu") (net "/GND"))
 (segment (start 67.4 79.2) (end 68.4 78.2) (width 0.6) (layer "B.Cu") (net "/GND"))
 (segment (start 67.4 30) (end 61.8 30) (width 0.6) (layer "B.Cu") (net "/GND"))
 (segment (start 68.4 31) (end 67.4 30) (width 0.6) (layer "B.Cu") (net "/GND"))
 (segment (start 9.8 39.9) (end 11.6 38.1) (width 0.6) (layer "B.Cu") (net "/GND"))
 (segment (start 37.3 72.7) (end 44.1 79.5) (width 0.6) (layer "B.Cu") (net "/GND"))
 (segment (start 68.4 56.4) (end 66.7 54.7) (width 0.6) (layer "B.Cu") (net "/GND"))
 (segment (start 68.4 52.9) (end 68.4 31) (width 0.6) (layer "B.Cu") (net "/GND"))
 (segment (start 5.8 54.6) (end 9.8 50.6) (width 0.6) (layer "B.Cu") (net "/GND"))
 (segment (start 53.3 79.2) (end 67.4 79.2) (width 0.6) (layer "B.Cu") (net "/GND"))
 (segment (start 11.6 38.1) (end 12 38.1) (width 0.6) (layer "B.Cu") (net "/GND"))
 (segment (start 61.8 30) (end 57.2 34.6) (width 0.6) (layer "B.Cu") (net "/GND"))
 (segment (start 34 39.7) (end 33.5 39.7) (width 0.6) (layer "F.Cu") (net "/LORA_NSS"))
 (segment (start 11 62.2) (end 11 63.9) (width 0.6) (layer "F.Cu") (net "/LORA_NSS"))
 (segment (start 33.5 39.7) (end 11 62.2) (width 0.6) (layer "F.Cu") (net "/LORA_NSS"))
 (segment (start 11 64.6) (end 5.8 69.8) (width 0.6) (layer "B.Cu") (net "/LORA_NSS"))
 (segment (start 11 63.9) (end 11 64.6) (width 0.6) (layer "B.Cu") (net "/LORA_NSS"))
 (segment (start 7.5 63.2) (end 7.5 70.6) (width 0.6) (layer "F.Cu") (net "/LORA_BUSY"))
 (segment (start 7.5 70.6) (end 5.8 72.3) (width 0.6) (layer "F.Cu") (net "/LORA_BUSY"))
 (segment (start 33.6 37.1) (end 7.5 63.2) (width 0.6) (layer "F.Cu") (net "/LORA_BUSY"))
 (segment (start 34 37.1) (end 33.6 37.1) (width 0.6) (layer "F.Cu") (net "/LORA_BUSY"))
 (segment (start 33.6 77.4) (end 5.8 77.4) (width 0.6) (layer "B.Cu") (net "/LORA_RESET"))
 (segment (start 34 77.8) (end 33.6 77.4) (width 0.6) (layer "B.Cu") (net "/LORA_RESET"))
 (segment (start 49 77.9) (end 50.5 79.4) (width 0.6) (layer "F.Cu") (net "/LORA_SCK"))
 (segment (start 52.7 79.4) (end 53 79.4) (width 0.6) (layer "F.Cu") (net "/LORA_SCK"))
 (segment (start 53 79.4) (end 53.9 78.5) (width 0.6) (layer "F.Cu") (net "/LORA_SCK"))
 (segment (start 53.9 78.3) (end 54 78.2) (width 0.6) (layer "F.Cu") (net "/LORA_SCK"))
 (segment (start 50.8 79.4) (end 50.9 79.5) (width 0.6) (layer "F.Cu") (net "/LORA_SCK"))
 (segment (start 50.5 79.4) (end 50.8 79.4) (width 0.6) (layer "F.Cu") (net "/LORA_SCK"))
 (segment (start 34.5 62.5) (end 49 77) (width 0.6) (layer "F.Cu") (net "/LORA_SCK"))
 (segment (start 52.6 79.5) (end 52.7 79.4) (width 0.6) (layer "F.Cu") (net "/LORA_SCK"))
 (segment (start 54 54.6) (end 64.2 44.4) (width 0.6) (layer "F.Cu") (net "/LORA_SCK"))
 (segment (start 50.9 79.5) (end 52.6 79.5) (width 0.6) (layer "F.Cu") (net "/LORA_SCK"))
 (segment (start 53.9 78.5) (end 53.9 78.3) (width 0.6) (layer "F.Cu") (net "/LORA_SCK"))
 (segment (start 54 78.2) (end 54 54.6) (width 0.6) (layer "F.Cu") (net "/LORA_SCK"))
 (segment (start 34 62.5) (end 34.5 62.5) (width 0.6) (layer "F.Cu") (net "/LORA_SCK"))
 (segment (start 49 77) (end 49 77.9) (width 0.6) (layer "F.Cu") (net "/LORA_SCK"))
 (segment (start 55.9 79.6) (end 55.9 79.3) (width 0.6) (layer "F.Cu") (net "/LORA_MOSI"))
 (segment (start 55.6 79.9) (end 55.9 79.6) (width 0.6) (layer "F.Cu") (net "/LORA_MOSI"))
 (segment (start 55.9 79.3) (end 56 79.2) (width 0.6) (layer "F.Cu") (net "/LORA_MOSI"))
 (segment (start 61.5 55.4) (end 62.5 54.4) (width 0.6) (layer "F.Cu") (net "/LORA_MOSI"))
 (segment (start 54.2 81.5) (end 55.6 80.1) (width 0.6) (layer "F.Cu") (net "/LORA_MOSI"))
 (segment (start 45 77.3) (end 49.2 81.5) (width 0.6) (layer "F.Cu") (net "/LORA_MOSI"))
 (segment (start 61.5 62.7) (end 61.5 55.4) (width 0.6) (layer "F.Cu") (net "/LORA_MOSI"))
 (segment (start 56 68.2) (end 61.5 62.7) (width 0.6) (layer "F.Cu") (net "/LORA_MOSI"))
 (segment (start 49.2 81.5) (end 54.2 81.5) (width 0.6) (layer "F.Cu") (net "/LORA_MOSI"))
 (segment (start 62.5 54.4) (end 62.5 51.2) (width 0.6) (layer "F.Cu") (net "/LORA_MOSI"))
 (segment (start 56 79.2) (end 56 68.2) (width 0.6) (layer "F.Cu") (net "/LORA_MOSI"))
 (segment (start 62.5 51.2) (end 64.2 49.5) (width 0.6) (layer "F.Cu") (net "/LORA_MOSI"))
 (segment (start 55.6 80.1) (end 55.6 79.9) (width 0.6) (layer "F.Cu") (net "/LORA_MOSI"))
 (segment (start 34 65.1) (end 34.5 65.1) (width 0.6) (layer "B.Cu") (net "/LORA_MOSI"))
 (segment (start 45 75.6) (end 45 77.3) (width 0.6) (layer "B.Cu") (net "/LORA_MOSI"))
 (segment (start 34.5 65.1) (end 45 75.6) (width 0.6) (layer "B.Cu") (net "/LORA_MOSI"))
 (segment (start 49.9 80.2) (end 49.7 80.2) (width 0.6) (layer "F.Cu") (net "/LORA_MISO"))
 (segment (start 49.7 80.2) (end 46.6 77.1) (width 0.6) (layer "F.Cu") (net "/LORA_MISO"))
 (segment (start 50.1 80.4) (end 49.9 80.2) (width 0.6) (layer "F.Cu") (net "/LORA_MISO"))
 (segment (start 53.1 80.5) (end 50.4 80.5) (width 0.6) (layer "F.Cu") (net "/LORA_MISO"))
 (segment (start 54.8 79.1) (end 54.8 79.3) (width 0.6) (layer "F.Cu") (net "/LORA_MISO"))
 (segment (start 57 61) (end 57 65.4) (width 0.6) (layer "F.Cu") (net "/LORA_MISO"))
 (segment (start 55 67.4) (end 55 78.7) (width 0.6) (layer "F.Cu") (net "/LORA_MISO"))
 (segment (start 53.9 80.1) (end 53.6 80.4) (width 0.6) (layer "F.Cu") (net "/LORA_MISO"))
 (segment (start 54.9 79) (end 54.8 79.1) (width 0.6) (layer "F.Cu") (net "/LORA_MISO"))
 (segment (start 46.6 76.837258) (end 45.662742 75.9) (width 0.6) (layer "F.Cu") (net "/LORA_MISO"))
 (segment (start 54 80.1) (end 53.9 80.1) (width 0.6) (layer "F.Cu") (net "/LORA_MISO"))
 (segment (start 50.3 80.4) (end 50.1 80.4) (width 0.6) (layer "F.Cu") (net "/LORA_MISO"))
 (segment (start 55 78.7) (end 54.9 78.8) (width 0.6) (layer "F.Cu") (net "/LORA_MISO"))
 (segment (start 54.8 79.3) (end 54 80.1) (width 0.6) (layer "F.Cu") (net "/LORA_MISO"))
 (segment (start 45.662742 75.9) (end 45.4 75.9) (width 0.6) (layer "F.Cu") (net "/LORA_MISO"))
 (segment (start 57 65.4) (end 55 67.4) (width 0.6) (layer "F.Cu") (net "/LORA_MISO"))
 (segment (start 37.1 67.6) (end 34 67.6) (width 0.6) (layer "F.Cu") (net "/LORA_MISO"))
 (segment (start 53.6 80.4) (end 53.2 80.4) (width 0.6) (layer "F.Cu") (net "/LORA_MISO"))
 (segment (start 46.6 77.1) (end 46.6 76.837258) (width 0.6) (layer "F.Cu") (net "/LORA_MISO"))
 (segment (start 50.4 80.5) (end 50.3 80.4) (width 0.6) (layer "F.Cu") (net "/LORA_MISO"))
 (segment (start 54.9 78.8) (end 54.9 79) (width 0.6) (layer "F.Cu") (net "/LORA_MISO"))
 (segment (start 45.4 75.9) (end 37.1 67.6) (width 0.6) (layer "F.Cu") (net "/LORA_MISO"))
 (segment (start 53.2 80.4) (end 53.1 80.5) (width 0.6) (layer "F.Cu") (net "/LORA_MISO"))
 (segment (start 55.2 59.2) (end 55.2 55.9) (width 0.6) (layer "B.Cu") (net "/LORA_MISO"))
 (segment (start 57 61) (end 55.2 59.2) (width 0.6) (layer "B.Cu") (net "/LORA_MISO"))
 (segment (start 55.2 55.9) (end 64.2 46.9) (width 0.6) (layer "B.Cu") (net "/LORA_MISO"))
 (segment (start 63.4 79.1) (end 67.5 79.1) (width 0.6) (layer "F.Cu") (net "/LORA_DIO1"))
 (segment (start 67.5 79.1) (end 68.4 78.2) (width 0.6) (layer "F.Cu") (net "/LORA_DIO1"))
 (segment (start 68.4 61.3) (end 66.7 59.6) (width 0.6) (layer "F.Cu") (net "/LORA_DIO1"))
 (segment (start 68.4 78.2) (end 68.4 61.3) (width 0.6) (layer "F.Cu") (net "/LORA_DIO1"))
 (segment (start 61.65 77.35) (end 63.4 79.1) (width 0.6) (layer "F.Cu") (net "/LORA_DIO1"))
 (segment (start 54 69.7) (end 54 66.8) (width 0.6) (layer "B.Cu") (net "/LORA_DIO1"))
 (segment (start 54 66.8) (end 52.3 65.1) (width 0.6) (layer "B.Cu") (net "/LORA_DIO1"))
 (segment (start 61.65 77.35) (end 54 69.7) (width 0.6) (layer "B.Cu") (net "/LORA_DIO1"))
 (segment (start 52.3 65.1) (end 51.8 65.1) (width 0.6) (layer "B.Cu") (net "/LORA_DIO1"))
 (segment (start 58 79.2) (end 62.5 74.7) (width 0.6) (layer "F.Cu") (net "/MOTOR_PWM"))
 (segment (start 62.5 61.3) (end 64.2 59.6) (width 0.6) (layer "F.Cu") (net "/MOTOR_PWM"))
 (segment (start 62.5 74.7) (end 62.5 61.3) (width 0.6) (layer "F.Cu") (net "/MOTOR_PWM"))
 (segment (start 59.5 81) (end 58 79.5) (width 0.6) (layer "F.Cu") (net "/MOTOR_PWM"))
 (segment (start 14 68.3) (end 14 68) (width 0.6) (layer "F.Cu") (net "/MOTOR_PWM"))
 (segment (start 24.7 79) (end 14 68.3) (width 0.6) (layer "F.Cu") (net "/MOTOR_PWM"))
 (segment (start 29.5 79) (end 24.7 79) (width 0.6) (layer "F.Cu") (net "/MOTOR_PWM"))
 (segment (start 58 79.5) (end 58 79.2) (width 0.6) (layer "F.Cu") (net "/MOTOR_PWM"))
 (segment (start 57.5 81) (end 57 80.5) (width 0.6) (layer "B.Cu") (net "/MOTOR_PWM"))
 (segment (start 33.6 80.5) (end 32.1 79) (width 0.6) (layer "B.Cu") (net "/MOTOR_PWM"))
 (segment (start 57 80.5) (end 33.6 80.5) (width 0.6) (layer "B.Cu") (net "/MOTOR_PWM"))
 (segment (start 32.1 79) (end 29.5 79) (width 0.6) (layer "B.Cu") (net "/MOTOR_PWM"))
 (segment (start 59.5 81) (end 57.5 81) (width 0.6) (layer "B.Cu") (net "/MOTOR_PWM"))
 (segment (start 12 40.6) (end 12.9 40.6) (width 0.6) (layer "F.Cu") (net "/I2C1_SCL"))
 (segment (start 12.9 40.6) (end 26.7 26.8) (width 0.6) (layer "F.Cu") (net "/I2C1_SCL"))
 (segment (start 56.8 26.8) (end 64.2 34.2) (width 0.6) (layer "F.Cu") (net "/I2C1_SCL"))
 (segment (start 26.7 26.8) (end 56.8 26.8) (width 0.6) (layer "F.Cu") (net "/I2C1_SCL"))
 (segment (start 12 43.2) (end 17.4 43.2) (width 0.6) (layer "F.Cu") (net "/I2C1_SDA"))
 (segment (start 32.8 27.8) (end 55.2 27.8) (width 0.6) (layer "F.Cu") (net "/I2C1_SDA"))
 (segment (start 17.4 43.2) (end 32.8 27.8) (width 0.6) (layer "F.Cu") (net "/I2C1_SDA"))
 (segment (start 55.2 27.8) (end 64.2 36.8) (width 0.6) (layer "F.Cu") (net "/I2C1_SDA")))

